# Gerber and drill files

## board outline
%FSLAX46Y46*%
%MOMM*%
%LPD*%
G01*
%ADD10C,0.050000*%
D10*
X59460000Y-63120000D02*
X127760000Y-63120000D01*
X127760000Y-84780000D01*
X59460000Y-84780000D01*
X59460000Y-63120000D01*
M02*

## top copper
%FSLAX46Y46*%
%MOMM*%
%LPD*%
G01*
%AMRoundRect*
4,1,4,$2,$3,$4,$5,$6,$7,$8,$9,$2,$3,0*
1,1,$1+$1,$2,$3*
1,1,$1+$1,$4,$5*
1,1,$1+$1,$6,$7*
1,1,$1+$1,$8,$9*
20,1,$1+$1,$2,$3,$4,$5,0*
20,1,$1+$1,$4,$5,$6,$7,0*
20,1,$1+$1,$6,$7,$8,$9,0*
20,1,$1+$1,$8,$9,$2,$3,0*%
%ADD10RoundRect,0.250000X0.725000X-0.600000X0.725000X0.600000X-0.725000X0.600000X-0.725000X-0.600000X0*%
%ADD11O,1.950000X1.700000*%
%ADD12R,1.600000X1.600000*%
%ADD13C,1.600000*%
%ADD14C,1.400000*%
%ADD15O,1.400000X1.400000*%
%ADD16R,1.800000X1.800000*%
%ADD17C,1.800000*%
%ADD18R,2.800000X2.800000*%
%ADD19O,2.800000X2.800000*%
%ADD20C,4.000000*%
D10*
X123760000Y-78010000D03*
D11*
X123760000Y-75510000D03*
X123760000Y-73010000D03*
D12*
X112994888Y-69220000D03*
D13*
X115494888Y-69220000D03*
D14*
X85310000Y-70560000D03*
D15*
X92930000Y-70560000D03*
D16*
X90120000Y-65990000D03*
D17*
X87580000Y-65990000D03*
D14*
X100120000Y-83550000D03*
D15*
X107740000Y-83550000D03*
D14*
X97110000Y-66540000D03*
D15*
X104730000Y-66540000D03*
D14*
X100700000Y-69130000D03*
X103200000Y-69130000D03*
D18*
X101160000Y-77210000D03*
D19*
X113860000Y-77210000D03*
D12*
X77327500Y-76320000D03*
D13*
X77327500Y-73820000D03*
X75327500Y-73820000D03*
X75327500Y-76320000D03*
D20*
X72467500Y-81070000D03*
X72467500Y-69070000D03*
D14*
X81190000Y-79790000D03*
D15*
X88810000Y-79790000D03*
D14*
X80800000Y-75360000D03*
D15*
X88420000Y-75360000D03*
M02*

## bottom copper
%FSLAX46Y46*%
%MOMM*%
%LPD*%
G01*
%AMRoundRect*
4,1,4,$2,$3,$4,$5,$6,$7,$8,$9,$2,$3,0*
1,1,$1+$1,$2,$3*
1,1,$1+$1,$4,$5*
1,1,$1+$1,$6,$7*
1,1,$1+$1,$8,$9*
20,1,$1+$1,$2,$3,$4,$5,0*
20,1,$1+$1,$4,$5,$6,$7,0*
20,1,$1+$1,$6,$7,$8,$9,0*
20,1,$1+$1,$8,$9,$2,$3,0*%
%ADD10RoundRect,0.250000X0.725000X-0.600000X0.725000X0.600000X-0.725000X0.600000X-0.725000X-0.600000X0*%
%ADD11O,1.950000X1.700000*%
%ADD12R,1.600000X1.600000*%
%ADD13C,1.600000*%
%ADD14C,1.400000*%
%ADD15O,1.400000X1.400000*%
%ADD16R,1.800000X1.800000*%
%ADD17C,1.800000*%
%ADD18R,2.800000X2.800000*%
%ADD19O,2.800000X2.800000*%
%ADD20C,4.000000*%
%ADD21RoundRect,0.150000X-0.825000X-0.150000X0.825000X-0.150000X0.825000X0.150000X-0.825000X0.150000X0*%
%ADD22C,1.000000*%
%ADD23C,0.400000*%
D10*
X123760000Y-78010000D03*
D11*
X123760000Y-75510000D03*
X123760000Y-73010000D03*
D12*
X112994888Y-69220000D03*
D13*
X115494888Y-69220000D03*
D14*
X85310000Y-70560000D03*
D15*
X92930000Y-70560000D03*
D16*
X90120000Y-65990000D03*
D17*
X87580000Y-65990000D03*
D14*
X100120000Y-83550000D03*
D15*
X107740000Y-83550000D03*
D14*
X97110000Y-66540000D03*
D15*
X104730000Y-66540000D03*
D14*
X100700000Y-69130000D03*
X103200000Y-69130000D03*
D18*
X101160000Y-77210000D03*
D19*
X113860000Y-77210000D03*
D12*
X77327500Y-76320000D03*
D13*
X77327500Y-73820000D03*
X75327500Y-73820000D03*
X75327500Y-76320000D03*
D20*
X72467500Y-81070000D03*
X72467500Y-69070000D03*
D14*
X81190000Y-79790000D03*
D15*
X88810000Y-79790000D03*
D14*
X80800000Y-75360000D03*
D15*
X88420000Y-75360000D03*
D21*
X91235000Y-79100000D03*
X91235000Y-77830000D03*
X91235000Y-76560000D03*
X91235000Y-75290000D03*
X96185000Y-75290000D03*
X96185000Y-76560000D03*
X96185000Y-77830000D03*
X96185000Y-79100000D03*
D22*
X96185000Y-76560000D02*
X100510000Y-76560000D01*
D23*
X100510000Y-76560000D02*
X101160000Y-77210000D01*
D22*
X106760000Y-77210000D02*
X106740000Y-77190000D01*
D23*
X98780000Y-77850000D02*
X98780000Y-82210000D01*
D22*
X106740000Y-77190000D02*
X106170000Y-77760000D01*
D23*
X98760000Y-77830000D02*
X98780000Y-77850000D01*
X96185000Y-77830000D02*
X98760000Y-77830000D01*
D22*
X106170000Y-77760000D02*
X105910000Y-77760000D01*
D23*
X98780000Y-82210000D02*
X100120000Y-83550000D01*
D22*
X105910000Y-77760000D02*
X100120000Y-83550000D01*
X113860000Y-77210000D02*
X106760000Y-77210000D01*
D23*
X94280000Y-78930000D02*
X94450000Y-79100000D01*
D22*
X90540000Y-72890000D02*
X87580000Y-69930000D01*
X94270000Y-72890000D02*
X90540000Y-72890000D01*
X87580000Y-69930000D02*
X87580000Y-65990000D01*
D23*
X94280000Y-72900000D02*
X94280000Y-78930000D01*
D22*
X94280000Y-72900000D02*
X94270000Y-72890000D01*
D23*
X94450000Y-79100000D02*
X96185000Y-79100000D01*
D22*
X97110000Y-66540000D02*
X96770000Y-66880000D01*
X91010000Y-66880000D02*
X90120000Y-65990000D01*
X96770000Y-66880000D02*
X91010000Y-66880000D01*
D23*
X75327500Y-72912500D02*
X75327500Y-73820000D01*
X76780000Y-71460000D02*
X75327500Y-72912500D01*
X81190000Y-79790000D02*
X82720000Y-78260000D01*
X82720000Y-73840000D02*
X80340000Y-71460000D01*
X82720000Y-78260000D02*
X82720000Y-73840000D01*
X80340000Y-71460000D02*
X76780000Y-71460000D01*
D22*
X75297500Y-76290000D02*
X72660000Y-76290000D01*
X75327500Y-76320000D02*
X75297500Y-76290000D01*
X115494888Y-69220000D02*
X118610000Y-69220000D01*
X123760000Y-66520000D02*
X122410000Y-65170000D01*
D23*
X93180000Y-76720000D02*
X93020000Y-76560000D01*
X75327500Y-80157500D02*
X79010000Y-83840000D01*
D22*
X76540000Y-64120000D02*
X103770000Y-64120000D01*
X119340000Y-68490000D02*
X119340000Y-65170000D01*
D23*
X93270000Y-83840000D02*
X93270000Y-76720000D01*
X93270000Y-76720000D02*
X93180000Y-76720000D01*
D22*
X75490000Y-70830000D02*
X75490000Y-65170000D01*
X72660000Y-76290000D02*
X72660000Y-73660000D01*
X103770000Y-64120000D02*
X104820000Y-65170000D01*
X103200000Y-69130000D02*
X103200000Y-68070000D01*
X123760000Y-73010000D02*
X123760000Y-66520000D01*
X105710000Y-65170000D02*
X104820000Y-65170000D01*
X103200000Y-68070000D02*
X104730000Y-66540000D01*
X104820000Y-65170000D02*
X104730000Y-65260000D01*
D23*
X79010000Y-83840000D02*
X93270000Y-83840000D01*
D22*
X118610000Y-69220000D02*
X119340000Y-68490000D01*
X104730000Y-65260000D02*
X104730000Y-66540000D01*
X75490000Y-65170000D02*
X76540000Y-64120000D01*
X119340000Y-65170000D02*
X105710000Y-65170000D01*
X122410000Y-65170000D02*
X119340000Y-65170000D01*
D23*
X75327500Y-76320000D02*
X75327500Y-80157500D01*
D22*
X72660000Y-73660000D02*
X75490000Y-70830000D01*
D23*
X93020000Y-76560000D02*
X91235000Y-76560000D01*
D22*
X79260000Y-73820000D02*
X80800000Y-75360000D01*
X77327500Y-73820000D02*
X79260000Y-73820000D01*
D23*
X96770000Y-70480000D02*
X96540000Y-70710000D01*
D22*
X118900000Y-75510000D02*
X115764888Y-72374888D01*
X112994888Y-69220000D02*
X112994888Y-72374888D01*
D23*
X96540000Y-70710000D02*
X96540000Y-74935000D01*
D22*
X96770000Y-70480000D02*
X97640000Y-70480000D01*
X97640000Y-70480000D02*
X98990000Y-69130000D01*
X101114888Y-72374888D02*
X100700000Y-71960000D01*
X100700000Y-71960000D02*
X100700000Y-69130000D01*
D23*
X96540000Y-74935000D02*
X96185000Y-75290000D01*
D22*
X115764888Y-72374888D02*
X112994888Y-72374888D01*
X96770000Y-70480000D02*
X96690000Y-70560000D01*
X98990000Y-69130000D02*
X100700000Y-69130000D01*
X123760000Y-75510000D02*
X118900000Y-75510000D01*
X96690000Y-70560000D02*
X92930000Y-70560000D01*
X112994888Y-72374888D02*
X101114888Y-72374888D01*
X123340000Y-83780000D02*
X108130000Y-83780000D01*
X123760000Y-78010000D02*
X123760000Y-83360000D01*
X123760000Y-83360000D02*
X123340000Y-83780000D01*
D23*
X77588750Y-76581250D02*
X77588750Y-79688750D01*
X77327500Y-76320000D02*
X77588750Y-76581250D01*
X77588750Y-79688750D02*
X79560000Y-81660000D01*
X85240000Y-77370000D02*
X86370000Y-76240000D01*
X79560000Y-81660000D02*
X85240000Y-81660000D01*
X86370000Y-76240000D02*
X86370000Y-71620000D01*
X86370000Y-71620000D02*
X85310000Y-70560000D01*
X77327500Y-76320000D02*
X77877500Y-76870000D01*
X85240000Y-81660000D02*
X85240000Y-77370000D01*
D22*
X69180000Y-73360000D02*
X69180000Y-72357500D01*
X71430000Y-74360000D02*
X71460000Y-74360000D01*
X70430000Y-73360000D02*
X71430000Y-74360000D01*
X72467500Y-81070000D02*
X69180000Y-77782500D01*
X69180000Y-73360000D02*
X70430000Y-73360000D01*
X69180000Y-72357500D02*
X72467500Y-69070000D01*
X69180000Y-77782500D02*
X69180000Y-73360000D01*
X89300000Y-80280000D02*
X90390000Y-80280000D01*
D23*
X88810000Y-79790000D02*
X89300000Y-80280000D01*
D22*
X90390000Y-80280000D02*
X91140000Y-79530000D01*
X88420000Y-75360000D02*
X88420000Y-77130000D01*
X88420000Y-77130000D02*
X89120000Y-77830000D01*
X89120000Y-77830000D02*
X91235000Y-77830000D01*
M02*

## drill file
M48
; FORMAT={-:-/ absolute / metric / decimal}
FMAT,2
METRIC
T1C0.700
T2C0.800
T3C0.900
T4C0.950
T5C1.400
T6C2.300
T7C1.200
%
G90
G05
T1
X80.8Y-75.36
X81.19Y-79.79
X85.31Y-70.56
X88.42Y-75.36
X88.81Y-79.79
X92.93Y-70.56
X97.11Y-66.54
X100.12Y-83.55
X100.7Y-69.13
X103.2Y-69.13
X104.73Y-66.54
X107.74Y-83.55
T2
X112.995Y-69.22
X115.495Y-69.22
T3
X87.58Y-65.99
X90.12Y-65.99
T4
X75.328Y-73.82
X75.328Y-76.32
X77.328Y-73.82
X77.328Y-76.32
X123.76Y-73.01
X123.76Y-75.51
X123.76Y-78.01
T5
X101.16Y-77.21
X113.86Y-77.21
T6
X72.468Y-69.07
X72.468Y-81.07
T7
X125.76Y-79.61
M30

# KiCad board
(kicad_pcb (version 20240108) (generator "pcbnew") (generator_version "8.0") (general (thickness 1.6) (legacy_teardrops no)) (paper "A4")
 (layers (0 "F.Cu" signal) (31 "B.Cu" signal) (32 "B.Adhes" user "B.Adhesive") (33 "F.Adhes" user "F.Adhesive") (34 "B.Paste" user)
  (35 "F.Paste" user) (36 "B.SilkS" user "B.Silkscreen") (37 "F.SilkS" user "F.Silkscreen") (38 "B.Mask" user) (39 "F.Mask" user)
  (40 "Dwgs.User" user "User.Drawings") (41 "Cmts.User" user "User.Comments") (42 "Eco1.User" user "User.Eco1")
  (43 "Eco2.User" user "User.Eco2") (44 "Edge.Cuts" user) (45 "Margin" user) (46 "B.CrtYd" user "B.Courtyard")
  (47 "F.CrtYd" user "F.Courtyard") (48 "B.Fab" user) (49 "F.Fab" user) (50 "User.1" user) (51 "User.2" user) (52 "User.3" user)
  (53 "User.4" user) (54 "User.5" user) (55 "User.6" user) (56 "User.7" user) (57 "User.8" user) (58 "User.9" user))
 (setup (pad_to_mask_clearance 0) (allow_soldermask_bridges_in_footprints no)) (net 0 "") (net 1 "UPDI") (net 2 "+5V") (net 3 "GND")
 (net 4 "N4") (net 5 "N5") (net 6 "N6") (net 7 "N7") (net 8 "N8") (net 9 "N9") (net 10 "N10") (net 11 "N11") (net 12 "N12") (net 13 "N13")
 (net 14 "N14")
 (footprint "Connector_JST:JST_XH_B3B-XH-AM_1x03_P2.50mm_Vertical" (layer "F.Cu") (at 123.76 78.01 90)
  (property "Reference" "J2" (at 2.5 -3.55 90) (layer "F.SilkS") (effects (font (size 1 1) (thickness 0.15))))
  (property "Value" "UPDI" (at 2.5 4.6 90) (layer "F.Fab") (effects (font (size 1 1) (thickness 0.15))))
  (pad "" np_thru_hole circle (at -1.6 2 90) (size 1.2 1.2) (drill 1.2) (layers "*.Cu" "*.Mask"))
  (pad "1" thru_hole roundrect (at 0 0 90) (size 1.7 1.95) (drill 0.95) (layers "*.Cu" "*.Mask") (remove_unused_layers no)
   (roundrect_rratio 0.147059) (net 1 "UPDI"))
  (pad "2" thru_hole oval (at 2.5 0 90) (size 1.7 1.95) (drill 0.95) (layers "*.Cu" "*.Mask") (remove_unused_layers no) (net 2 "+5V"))
  (pad "3" thru_hole oval (at 5 0 90) (size 1.7 1.95) (drill 0.95) (layers "*.Cu" "*.Mask") (remove_unused_layers no) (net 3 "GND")))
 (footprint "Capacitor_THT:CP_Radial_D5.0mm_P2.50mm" (layer "F.Cu") (at 112.994888 69.22)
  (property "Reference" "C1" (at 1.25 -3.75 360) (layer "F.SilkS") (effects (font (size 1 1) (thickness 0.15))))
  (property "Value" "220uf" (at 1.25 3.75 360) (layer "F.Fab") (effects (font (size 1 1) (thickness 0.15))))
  (pad "1" thru_hole rect (at 0 0) (size 1.6 1.6) (drill 0.8) (layers "*.Cu" "*.Mask") (remove_unused_layers no) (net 2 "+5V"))
  (pad "2" thru_hole circle (at 2.5 0) (size 1.6 1.6) (drill 0.8) (layers "*.Cu" "*.Mask") (remove_unused_layers no) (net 3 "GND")))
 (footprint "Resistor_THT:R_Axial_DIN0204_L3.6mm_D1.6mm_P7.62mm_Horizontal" (layer "F.Cu") (at 85.31 70.56)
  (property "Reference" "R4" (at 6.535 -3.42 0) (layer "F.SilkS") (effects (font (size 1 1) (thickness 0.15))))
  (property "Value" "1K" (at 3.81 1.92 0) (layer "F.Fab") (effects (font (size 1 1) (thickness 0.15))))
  (pad "1" thru_hole circle (at 0 0) (size 1.4 1.4) (drill 0.7) (layers "*.Cu" "*.Mask") (remove_unused_layers no) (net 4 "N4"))
  (pad "2" thru_hole oval (at 7.62 0) (size 1.4 1.4) (drill 0.7) (layers "*.Cu" "*.Mask") (remove_unused_layers no) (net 2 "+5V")))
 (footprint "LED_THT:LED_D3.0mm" (layer "F.Cu") (at 90.12 65.99 180)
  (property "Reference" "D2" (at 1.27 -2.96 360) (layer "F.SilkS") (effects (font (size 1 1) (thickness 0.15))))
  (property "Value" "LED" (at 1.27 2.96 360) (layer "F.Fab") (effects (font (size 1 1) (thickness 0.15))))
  (pad "1" thru_hole rect (at 0 0 180) (size 1.8 1.8) (drill 0.9) (layers "*.Cu" "*.Mask") (remove_unused_layers no) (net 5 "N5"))
  (pad "2" thru_hole circle (at 2.54 0 180) (size 1.8 1.8) (drill 0.9) (layers "*.Cu" "*.Mask") (remove_unused_layers no) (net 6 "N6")))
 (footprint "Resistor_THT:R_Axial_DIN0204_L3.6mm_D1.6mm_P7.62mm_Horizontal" (layer "F.Cu") (at 100.12 83.55)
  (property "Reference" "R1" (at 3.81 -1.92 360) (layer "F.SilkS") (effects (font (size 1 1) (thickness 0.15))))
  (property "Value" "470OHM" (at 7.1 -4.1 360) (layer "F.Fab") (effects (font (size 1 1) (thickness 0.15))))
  (pad "1" thru_hole circle (at 0 0) (size 1.4 1.4) (drill 0.7) (layers "*.Cu" "*.Mask") (remove_unused_layers no) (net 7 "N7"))
  (pad "2" thru_hole oval (at 7.62 0) (size 1.4 1.4) (drill 0.7) (layers "*.Cu" "*.Mask") (remove_unused_layers no) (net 1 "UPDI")))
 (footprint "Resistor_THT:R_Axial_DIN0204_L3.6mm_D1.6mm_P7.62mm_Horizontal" (layer "F.Cu") (at 97.11 66.54)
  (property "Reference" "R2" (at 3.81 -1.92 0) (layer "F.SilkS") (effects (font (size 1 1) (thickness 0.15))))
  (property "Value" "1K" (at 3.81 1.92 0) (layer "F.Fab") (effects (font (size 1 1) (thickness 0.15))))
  (pad "1" thru_hole circle (at 0 0) (size 1.4 1.4) (drill 0.7) (layers "*.Cu" "*.Mask") (remove_unused_layers no) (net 5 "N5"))
  (pad "2" thru_hole oval (at 7.62 0) (size 1.4 1.4) (drill 0.7) (layers "*.Cu" "*.Mask") (remove_unused_layers no) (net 3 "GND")))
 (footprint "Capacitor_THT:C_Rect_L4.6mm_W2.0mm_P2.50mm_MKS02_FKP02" (layer "F.Cu") (at 100.7 69.13)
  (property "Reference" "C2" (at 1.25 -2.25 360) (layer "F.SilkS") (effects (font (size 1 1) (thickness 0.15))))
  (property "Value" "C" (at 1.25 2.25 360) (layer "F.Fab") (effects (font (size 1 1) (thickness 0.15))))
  (pad "1" thru_hole circle (at 0 0) (size 1.4 1.4) (drill 0.7) (layers "*.Cu" "*.Mask") (remove_unused_layers no) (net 2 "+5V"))
  (pad "2" thru_hole circle (at 2.5 0) (size 1.4 1.4) (drill 0.7) (layers "*.Cu" "*.Mask") (remove_unused_layers no) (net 3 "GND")))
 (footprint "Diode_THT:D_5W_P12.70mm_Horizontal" (layer "F.Cu") (at 101.16 77.21)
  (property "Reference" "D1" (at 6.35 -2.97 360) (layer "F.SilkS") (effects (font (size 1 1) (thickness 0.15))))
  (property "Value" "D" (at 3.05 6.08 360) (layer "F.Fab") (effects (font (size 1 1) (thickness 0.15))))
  (pad "1" thru_hole rect (at 0 0) (size 2.8 2.8) (drill 1.4) (layers "*.Cu" "*.Mask") (remove_unused_layers no) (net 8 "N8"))
  (pad "2" thru_hole oval (at 12.7 0) (size 2.8 2.8) (drill 1.4) (layers "*.Cu" "*.Mask") (remove_unused_layers no) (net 7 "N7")))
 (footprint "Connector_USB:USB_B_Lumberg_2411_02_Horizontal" (layer "F.Cu") (at 77.3275 76.32 180)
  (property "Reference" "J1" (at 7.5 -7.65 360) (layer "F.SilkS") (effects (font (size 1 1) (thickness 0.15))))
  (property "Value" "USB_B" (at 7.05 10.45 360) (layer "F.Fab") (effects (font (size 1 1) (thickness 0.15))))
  (pad "1" thru_hole rect (at 0 0 270) (size 1.6 1.6) (drill 0.95) (layers "*.Cu" "*.Mask") (remove_unused_layers no) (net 4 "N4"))
  (pad "2" thru_hole circle (at 0 2.5 270) (size 1.6 1.6) (drill 0.95) (layers "*.Cu" "*.Mask") (remove_unused_layers no) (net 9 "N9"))
  (pad "3" thru_hole circle (at 2 2.5 270) (size 1.6 1.6) (drill 0.95) (layers "*.Cu" "*.Mask") (remove_unused_layers no) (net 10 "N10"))
  (pad "4" thru_hole circle (at 2 0 270) (size 1.6 1.6) (drill 0.95) (layers "*.Cu" "*.Mask") (remove_unused_layers no) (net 3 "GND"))
  (pad "5" thru_hole circle (at 4.86 -4.75 270) (size 4 4) (drill 2.3) (layers "*.Cu" "*.Mask") (remove_unused_layers no) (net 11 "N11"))
  (pad "5" thru_hole circle (at 4.86 7.25 270) (size 4 4) (drill 2.3) (layers "*.Cu" "*.Mask") (remove_unused_layers no) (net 11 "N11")))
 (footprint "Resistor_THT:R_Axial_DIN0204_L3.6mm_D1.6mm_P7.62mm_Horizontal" (layer "F.Cu") (at 81.19 79.79)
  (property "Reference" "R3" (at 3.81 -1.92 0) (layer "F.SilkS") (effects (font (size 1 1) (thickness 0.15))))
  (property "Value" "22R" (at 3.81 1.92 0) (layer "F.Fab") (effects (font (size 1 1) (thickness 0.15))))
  (pad "1" thru_hole circle (at 0 0) (size 1.4 1.4) (drill 0.7) (layers "*.Cu" "*.Mask") (remove_unused_layers no) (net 10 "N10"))
  (pad "2" thru_hole oval (at 7.62 0) (size 1.4 1.4) (drill 0.7) (layers "*.Cu" "*.Mask") (remove_unused_layers no) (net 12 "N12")))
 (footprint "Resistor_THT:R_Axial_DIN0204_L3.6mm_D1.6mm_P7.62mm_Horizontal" (layer "F.Cu") (at 80.8 75.36)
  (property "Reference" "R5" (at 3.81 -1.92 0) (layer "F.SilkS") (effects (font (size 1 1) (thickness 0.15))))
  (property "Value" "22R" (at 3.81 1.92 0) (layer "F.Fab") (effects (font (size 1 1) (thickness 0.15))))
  (pad "1" thru_hole circle (at 0 0) (size 1.4 1.4) (drill 0.7) (layers "*.Cu" "*.Mask") (remove_unused_layers no) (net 9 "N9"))
  (pad "2" thru_hole oval (at 7.62 0) (size 1.4 1.4) (drill 0.7) (layers "*.Cu" "*.Mask") (remove_unused_layers no) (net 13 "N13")))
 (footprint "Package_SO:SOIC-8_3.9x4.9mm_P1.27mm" (layer "B.Cu") (at 93.71 77.195)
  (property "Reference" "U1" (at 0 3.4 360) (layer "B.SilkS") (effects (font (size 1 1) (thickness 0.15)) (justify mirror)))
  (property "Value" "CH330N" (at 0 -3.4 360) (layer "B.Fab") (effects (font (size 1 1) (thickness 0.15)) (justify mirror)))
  (pad "1" smd roundrect (at -2.475 1.905) (size 1.95 0.6) (layers "B.Cu" "B.Paste" "B.Mask") (roundrect_rratio 0.25) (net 12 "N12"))
  (pad "2" smd roundrect (at -2.475 0.635) (size 1.95 0.6) (layers "B.Cu" "B.Paste" "B.Mask") (roundrect_rratio 0.25) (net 13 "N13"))
  (pad "3" smd roundrect (at -2.475 -0.635) (size 1.95 0.6) (layers "B.Cu" "B.Paste" "B.Mask") (roundrect_rratio 0.25) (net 3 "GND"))
  (pad "4" smd roundrect (at -2.475 -1.905) (size 1.95 0.6) (layers "B.Cu" "B.Paste" "B.Mask") (roundrect_rratio 0.25) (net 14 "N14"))
  (pad "5" smd roundrect (at 2.475 -1.905) (size 1.95 0.6) (layers "B.Cu" "B.Paste" "B.Mask") (roundrect_rratio 0.25) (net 2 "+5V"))
  (pad "6" smd roundrect (at 2.475 -0.635) (size 1.95 0.6) (layers "B.Cu" "B.Paste" "B.Mask") (roundrect_rratio 0.25) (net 8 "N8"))
  (pad "7" smd roundrect (at 2.475 0.635) (size 1.95 0.6) (layers "B.Cu" "B.Paste" "B.Mask") (roundrect_rratio 0.25) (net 7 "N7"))
  (pad "8" smd roundrect (at 2.475 1.905) (size 1.95 0.6) (layers "B.Cu" "B.Paste" "B.Mask") (roundrect_rratio 0.25) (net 6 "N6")))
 (gr_rect (start 59.46 63.12) (end 127.76 84.78) (stroke (width 0.05) (type default)) (fill none) (layer "Edge.Cuts"))
 (segment (start 96.185 76.56) (end 100.51 76.56) (width 1) (layer "B.Cu") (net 8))
 (segment (start 100.51 76.56) (end 101.16 77.21) (width 0.4) (layer "B.Cu") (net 8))
 (segment (start 106.76 77.21) (end 106.74 77.19) (width 1) (layer "B.Cu") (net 7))
 (segment (start 98.78 77.85) (end 98.78 82.21) (width 0.4) (layer "B.Cu") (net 7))
 (segment (start 106.74 77.19) (end 106.17 77.76) (width 1) (layer "B.Cu") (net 7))
 (segment (start 98.76 77.83) (end 98.78 77.85) (width 0.4) (layer "B.Cu") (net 7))
 (segment (start 96.185 77.83) (end 98.76 77.83) (width 0.4) (layer "B.Cu") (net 7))
 (segment (start 106.17 77.76) (end 105.91 77.76) (width 1) (layer "B.Cu") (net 7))
 (segment (start 98.78 82.21) (end 100.12 83.55) (width 0.4) (layer "B.Cu") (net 7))
 (segment (start 105.91 77.76) (end 100.12 83.55) (width 1) (layer "B.Cu") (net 7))
 (segment (start 113.86 77.21) (end 106.76 77.21) (width 1) (layer "B.Cu") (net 7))
 (segment (start 94.28 78.93) (end 94.45 79.1) (width 0.4) (layer "B.Cu") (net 6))
 (segment (start 90.54 72.89) (end 87.58 69.93) (width 1) (layer "B.Cu") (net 6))
 (segment (start 94.27 72.89) (end 90.54 72.89) (width 1) (layer "B.Cu") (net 6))
 (segment (start 87.58 69.93) (end 87.58 65.99) (width 1) (layer "B.Cu") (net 6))
 (segment (start 94.28 72.9) (end 94.28 78.93) (width 0.4) (layer "B.Cu") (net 6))
 (segment (start 94.28 72.9) (end 94.27 72.89) (width 1) (layer "B.Cu") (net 6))
 (segment (start 94.45 79.1) (end 96.185 79.1) (width 0.4) (layer "B.Cu") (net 6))
 (segment (start 97.11 66.54) (end 96.77 66.88) (width 1) (layer "B.Cu") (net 5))
 (segment (start 91.01 66.88) (end 90.12 65.99) (width 1) (layer "B.Cu") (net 5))
 (segment (start 96.77 66.88) (end 91.01 66.88) (width 1) (layer "B.Cu") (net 5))
 (segment (start 75.3275 72.9125) (end 75.3275 73.82) (width 0.4) (layer "B.Cu") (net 10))
 (segment (start 76.78 71.46) (end 75.3275 72.9125) (width 0.4) (layer "B.Cu") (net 10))
 (segment (start 81.19 79.79) (end 82.72 78.26) (width 0.4) (layer "B.Cu") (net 10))
 (segment (start 82.72 73.84) (end 80.34 71.46) (width 0.4) (layer "B.Cu") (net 10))
 (segment (start 82.72 78.26) (end 82.72 73.84) (width 0.4) (layer "B.Cu") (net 10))
 (segment (start 80.34 71.46) (end 76.78 71.46) (width 0.4) (layer "B.Cu") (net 10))
 (segment (start 75.2975 76.29) (end 72.66 76.29) (width 1) (layer "B.Cu") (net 3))
 (segment (start 75.3275 76.32) (end 75.2975 76.29) (width 1) (layer "B.Cu") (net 3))
 (segment (start 115.494888 69.22) (end 118.61 69.22) (width 1) (layer "B.Cu") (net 3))
 (segment (start 123.76 66.52) (end 122.41 65.17) (width 1) (layer "B.Cu") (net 3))
 (segment (start 93.18 76.72) (end 93.02 76.56) (width 0.4) (layer "B.Cu") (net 3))
 (segment (start 75.3275 80.1575) (end 79.01 83.84) (width 0.4) (layer "B.Cu") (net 3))
 (segment (start 76.54 64.12) (end 103.77 64.12) (width 1) (layer "B.Cu") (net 3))
 (segment (start 119.34 68.49) (end 119.34 65.17) (width 1) (layer "B.Cu") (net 3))
 (segment (start 93.27 83.84) (end 93.27 76.72) (width 0.4) (layer "B.Cu") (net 3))
 (segment (start 93.27 76.72) (end 93.18 76.72) (width 0.4) (layer "B.Cu") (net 3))
 (segment (start 75.49 70.83) (end 75.49 65.17) (width 1) (layer "B.Cu") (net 3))
 (segment (start 72.66 76.29) (end 72.66 73.66) (width 1) (layer "B.Cu") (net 3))
 (segment (start 103.77 64.12) (end 104.82 65.17) (width 1) (layer "B.Cu") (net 3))
 (segment (start 103.2 69.13) (end 103.2 68.07) (width 1) (layer "B.Cu") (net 3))
 (segment (start 123.76 73.01) (end 123.76 66.52) (width 1) (layer "B.Cu") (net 3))
 (segment (start 105.71 65.17) (end 104.82 65.17) (width 1) (layer "B.Cu") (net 3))
 (segment (start 103.2 68.07) (end 104.73 66.54) (width 1) (layer "B.Cu") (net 3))
 (segment (start 104.82 65.17) (end 104.73 65.26) (width 1) (layer "B.Cu") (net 3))
 (segment (start 79.01 83.84) (end 93.27 83.84) (width 0.4) (layer "B.Cu") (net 3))
 (segment (start 118.61 69.22) (end 119.34 68.49) (width 1) (layer "B.Cu") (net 3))
 (segment (start 104.73 65.26) (end 104.73 66.54) (width 1) (layer "B.Cu") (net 3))
 (segment (start 75.49 65.17) (end 76.54 64.12) (width 1) (layer "B.Cu") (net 3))
 (segment (start 119.34 65.17) (end 105.71 65.17) (width 1) (layer "B.Cu") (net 3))
 (segment (start 122.41 65.17) (end 119.34 65.17) (width 1) (layer "B.Cu") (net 3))
 (segment (start 75.3275 76.32) (end 75.3275 80.1575) (width 0.4) (layer "B.Cu") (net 3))
 (segment (start 72.66 73.66) (end 75.49 70.83) (width 1) (layer "B.Cu") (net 3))
 (segment (start 93.02 76.56) (end 91.235 76.56) (width 0.4) (layer "B.Cu") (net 3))
 (segment (start 79.26 73.82) (end 80.8 75.36) (width 1) (layer "B.Cu") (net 9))
 (segment (start 77.3275 73.82) (end 79.26 73.82) (width 1) (layer "B.Cu") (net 9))
 (segment (start 96.77 70.48) (end 96.54 70.71) (width 0.4) (layer "B.Cu") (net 2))
 (segment (start 118.9 75.51) (end 115.764888 72.374888) (width 1) (layer "B.Cu") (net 2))
 (segment (start 112.994888 69.22) (end 112.994888 72.374888) (width 1) (layer "B.Cu") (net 2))
 (segment (start 96.54 70.71) (end 96.54 74.935) (width 0.4) (layer "B.Cu") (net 2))
 (segment (start 96.77 70.48) (end 97.64 70.48) (width 1) (layer "B.Cu") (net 2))
 (segment (start 97.64 70.48) (end 98.99 69.13) (width 1) (layer "B.Cu") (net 2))
 (segment (start 101.114888 72.374888) (end 100.7 71.96) (width 1) (layer "B.Cu") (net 2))
 (segment (start 100.7 71.96) (end 100.7 69.13) (width 1) (layer "B.Cu") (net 2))
 (segment (start 96.54 74.935) (end 96.185 75.29) (width 0.4) (layer "B.Cu") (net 2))
 (segment (start 115.764888 72.374888) (end 112.994888 72.374888) (width 1) (layer "B.Cu") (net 2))
 (segment (start 96.77 70.48) (end 96.69 70.56) (width 1) (layer "B.Cu") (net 2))
 (segment (start 98.99 69.13) (end 100.7 69.13) (width 1) (layer "B.Cu") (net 2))
 (segment (start 123.76 75.51) (end 118.9 75.51) (width 1) (layer "B.Cu") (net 2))
 (segment (start 96.69 70.56) (end 92.93 70.56) (width 1) (layer "B.Cu") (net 2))
 (segment (start 112.994888 72.374888) (end 101.114888 72.374888) (width 1) (layer "B.Cu") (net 2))
 (segment (start 123.34 83.78) (end 108.13 83.78) (width 1) (layer "B.Cu") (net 1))
 (segment (start 123.76 78.01) (end 123.76 83.36) (width 1) (layer "B.Cu") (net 1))
 (segment (start 123.76 83.36) (end 123.34 83.78) (width 1) (layer "B.Cu") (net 1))
 (segment (start 77.58875 76.58125) (end 77.58875 79.68875) (width 0.4) (layer "B.Cu") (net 4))
 (segment (start 77.3275 76.32) (end 77.58875 76.58125) (width 0.4) (layer "B.Cu") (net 4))
 (segment (start 77.58875 79.68875) (end 79.56 81.66) (width 0.4) (layer "B.Cu") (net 4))
 (segment (start 85.24 77.37) (end 86.37 76.24) (width 0.4) (layer "B.Cu") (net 4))
 (segment (start 79.56 81.66) (end 85.24 81.66) (width 0.4) (layer "B.Cu") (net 4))
 (segment (start 86.37 76.24) (end 86.37 71.62) (width 0.4) (layer "B.Cu") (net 4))
 (segment (start 86.37 71.62) (end 85.31 70.56) (width 0.4) (layer "B.Cu") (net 4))
 (segment (start 77.3275 76.32) (end 77.8775 76.87) (width 0.4) (layer "B.Cu") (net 4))
 (segment (start 85.24 81.66) (end 85.24 77.37) (width 0.4) (layer "B.Cu") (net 4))
 (segment (start 69.18 73.36) (end 69.18 72.3575) (width 1) (layer "B.Cu") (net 11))
 (segment (start 71.43 74.36) (end 71.46 74.36) (width 1) (layer "B.Cu") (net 11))
 (segment (start 70.43 73.36) (end 71.43 74.36) (width 1) (layer "B.Cu") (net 11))
 (segment (start 72.4675 81.07) (end 69.18 77.7825) (width 1) (layer "B.Cu") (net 11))
 (segment (start 69.18 73.36) (end 70.43 73.36) (width 1) (layer "B.Cu") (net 11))
 (segment (start 69.18 72.3575) (end 72.4675 69.07) (width 1) (layer "B.Cu") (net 11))
 (segment (start 69.18 77.7825) (end 69.18 73.36) (width 1) (layer "B.Cu") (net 11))
 (segment (start 89.3 80.28) (end 90.39 80.28) (width 1) (layer "B.Cu") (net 12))
 (segment (start 88.81 79.79) (end 89.3 80.28) (width 0.4) (layer "B.Cu") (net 12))
 (segment (start 90.39 80.28) (end 91.14 79.53) (width 1) (layer "B.Cu") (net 12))
 (segment (start 88.42 75.36) (end 88.42 77.13) (width 1) (layer "B.Cu") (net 13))
 (segment (start 88.42 77.13) (end 89.12 77.83) (width 1) (layer "B.Cu") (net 13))
 (segment (start 89.12 77.83) (end 91.235 77.83) (width 1) (layer "B.Cu") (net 13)))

